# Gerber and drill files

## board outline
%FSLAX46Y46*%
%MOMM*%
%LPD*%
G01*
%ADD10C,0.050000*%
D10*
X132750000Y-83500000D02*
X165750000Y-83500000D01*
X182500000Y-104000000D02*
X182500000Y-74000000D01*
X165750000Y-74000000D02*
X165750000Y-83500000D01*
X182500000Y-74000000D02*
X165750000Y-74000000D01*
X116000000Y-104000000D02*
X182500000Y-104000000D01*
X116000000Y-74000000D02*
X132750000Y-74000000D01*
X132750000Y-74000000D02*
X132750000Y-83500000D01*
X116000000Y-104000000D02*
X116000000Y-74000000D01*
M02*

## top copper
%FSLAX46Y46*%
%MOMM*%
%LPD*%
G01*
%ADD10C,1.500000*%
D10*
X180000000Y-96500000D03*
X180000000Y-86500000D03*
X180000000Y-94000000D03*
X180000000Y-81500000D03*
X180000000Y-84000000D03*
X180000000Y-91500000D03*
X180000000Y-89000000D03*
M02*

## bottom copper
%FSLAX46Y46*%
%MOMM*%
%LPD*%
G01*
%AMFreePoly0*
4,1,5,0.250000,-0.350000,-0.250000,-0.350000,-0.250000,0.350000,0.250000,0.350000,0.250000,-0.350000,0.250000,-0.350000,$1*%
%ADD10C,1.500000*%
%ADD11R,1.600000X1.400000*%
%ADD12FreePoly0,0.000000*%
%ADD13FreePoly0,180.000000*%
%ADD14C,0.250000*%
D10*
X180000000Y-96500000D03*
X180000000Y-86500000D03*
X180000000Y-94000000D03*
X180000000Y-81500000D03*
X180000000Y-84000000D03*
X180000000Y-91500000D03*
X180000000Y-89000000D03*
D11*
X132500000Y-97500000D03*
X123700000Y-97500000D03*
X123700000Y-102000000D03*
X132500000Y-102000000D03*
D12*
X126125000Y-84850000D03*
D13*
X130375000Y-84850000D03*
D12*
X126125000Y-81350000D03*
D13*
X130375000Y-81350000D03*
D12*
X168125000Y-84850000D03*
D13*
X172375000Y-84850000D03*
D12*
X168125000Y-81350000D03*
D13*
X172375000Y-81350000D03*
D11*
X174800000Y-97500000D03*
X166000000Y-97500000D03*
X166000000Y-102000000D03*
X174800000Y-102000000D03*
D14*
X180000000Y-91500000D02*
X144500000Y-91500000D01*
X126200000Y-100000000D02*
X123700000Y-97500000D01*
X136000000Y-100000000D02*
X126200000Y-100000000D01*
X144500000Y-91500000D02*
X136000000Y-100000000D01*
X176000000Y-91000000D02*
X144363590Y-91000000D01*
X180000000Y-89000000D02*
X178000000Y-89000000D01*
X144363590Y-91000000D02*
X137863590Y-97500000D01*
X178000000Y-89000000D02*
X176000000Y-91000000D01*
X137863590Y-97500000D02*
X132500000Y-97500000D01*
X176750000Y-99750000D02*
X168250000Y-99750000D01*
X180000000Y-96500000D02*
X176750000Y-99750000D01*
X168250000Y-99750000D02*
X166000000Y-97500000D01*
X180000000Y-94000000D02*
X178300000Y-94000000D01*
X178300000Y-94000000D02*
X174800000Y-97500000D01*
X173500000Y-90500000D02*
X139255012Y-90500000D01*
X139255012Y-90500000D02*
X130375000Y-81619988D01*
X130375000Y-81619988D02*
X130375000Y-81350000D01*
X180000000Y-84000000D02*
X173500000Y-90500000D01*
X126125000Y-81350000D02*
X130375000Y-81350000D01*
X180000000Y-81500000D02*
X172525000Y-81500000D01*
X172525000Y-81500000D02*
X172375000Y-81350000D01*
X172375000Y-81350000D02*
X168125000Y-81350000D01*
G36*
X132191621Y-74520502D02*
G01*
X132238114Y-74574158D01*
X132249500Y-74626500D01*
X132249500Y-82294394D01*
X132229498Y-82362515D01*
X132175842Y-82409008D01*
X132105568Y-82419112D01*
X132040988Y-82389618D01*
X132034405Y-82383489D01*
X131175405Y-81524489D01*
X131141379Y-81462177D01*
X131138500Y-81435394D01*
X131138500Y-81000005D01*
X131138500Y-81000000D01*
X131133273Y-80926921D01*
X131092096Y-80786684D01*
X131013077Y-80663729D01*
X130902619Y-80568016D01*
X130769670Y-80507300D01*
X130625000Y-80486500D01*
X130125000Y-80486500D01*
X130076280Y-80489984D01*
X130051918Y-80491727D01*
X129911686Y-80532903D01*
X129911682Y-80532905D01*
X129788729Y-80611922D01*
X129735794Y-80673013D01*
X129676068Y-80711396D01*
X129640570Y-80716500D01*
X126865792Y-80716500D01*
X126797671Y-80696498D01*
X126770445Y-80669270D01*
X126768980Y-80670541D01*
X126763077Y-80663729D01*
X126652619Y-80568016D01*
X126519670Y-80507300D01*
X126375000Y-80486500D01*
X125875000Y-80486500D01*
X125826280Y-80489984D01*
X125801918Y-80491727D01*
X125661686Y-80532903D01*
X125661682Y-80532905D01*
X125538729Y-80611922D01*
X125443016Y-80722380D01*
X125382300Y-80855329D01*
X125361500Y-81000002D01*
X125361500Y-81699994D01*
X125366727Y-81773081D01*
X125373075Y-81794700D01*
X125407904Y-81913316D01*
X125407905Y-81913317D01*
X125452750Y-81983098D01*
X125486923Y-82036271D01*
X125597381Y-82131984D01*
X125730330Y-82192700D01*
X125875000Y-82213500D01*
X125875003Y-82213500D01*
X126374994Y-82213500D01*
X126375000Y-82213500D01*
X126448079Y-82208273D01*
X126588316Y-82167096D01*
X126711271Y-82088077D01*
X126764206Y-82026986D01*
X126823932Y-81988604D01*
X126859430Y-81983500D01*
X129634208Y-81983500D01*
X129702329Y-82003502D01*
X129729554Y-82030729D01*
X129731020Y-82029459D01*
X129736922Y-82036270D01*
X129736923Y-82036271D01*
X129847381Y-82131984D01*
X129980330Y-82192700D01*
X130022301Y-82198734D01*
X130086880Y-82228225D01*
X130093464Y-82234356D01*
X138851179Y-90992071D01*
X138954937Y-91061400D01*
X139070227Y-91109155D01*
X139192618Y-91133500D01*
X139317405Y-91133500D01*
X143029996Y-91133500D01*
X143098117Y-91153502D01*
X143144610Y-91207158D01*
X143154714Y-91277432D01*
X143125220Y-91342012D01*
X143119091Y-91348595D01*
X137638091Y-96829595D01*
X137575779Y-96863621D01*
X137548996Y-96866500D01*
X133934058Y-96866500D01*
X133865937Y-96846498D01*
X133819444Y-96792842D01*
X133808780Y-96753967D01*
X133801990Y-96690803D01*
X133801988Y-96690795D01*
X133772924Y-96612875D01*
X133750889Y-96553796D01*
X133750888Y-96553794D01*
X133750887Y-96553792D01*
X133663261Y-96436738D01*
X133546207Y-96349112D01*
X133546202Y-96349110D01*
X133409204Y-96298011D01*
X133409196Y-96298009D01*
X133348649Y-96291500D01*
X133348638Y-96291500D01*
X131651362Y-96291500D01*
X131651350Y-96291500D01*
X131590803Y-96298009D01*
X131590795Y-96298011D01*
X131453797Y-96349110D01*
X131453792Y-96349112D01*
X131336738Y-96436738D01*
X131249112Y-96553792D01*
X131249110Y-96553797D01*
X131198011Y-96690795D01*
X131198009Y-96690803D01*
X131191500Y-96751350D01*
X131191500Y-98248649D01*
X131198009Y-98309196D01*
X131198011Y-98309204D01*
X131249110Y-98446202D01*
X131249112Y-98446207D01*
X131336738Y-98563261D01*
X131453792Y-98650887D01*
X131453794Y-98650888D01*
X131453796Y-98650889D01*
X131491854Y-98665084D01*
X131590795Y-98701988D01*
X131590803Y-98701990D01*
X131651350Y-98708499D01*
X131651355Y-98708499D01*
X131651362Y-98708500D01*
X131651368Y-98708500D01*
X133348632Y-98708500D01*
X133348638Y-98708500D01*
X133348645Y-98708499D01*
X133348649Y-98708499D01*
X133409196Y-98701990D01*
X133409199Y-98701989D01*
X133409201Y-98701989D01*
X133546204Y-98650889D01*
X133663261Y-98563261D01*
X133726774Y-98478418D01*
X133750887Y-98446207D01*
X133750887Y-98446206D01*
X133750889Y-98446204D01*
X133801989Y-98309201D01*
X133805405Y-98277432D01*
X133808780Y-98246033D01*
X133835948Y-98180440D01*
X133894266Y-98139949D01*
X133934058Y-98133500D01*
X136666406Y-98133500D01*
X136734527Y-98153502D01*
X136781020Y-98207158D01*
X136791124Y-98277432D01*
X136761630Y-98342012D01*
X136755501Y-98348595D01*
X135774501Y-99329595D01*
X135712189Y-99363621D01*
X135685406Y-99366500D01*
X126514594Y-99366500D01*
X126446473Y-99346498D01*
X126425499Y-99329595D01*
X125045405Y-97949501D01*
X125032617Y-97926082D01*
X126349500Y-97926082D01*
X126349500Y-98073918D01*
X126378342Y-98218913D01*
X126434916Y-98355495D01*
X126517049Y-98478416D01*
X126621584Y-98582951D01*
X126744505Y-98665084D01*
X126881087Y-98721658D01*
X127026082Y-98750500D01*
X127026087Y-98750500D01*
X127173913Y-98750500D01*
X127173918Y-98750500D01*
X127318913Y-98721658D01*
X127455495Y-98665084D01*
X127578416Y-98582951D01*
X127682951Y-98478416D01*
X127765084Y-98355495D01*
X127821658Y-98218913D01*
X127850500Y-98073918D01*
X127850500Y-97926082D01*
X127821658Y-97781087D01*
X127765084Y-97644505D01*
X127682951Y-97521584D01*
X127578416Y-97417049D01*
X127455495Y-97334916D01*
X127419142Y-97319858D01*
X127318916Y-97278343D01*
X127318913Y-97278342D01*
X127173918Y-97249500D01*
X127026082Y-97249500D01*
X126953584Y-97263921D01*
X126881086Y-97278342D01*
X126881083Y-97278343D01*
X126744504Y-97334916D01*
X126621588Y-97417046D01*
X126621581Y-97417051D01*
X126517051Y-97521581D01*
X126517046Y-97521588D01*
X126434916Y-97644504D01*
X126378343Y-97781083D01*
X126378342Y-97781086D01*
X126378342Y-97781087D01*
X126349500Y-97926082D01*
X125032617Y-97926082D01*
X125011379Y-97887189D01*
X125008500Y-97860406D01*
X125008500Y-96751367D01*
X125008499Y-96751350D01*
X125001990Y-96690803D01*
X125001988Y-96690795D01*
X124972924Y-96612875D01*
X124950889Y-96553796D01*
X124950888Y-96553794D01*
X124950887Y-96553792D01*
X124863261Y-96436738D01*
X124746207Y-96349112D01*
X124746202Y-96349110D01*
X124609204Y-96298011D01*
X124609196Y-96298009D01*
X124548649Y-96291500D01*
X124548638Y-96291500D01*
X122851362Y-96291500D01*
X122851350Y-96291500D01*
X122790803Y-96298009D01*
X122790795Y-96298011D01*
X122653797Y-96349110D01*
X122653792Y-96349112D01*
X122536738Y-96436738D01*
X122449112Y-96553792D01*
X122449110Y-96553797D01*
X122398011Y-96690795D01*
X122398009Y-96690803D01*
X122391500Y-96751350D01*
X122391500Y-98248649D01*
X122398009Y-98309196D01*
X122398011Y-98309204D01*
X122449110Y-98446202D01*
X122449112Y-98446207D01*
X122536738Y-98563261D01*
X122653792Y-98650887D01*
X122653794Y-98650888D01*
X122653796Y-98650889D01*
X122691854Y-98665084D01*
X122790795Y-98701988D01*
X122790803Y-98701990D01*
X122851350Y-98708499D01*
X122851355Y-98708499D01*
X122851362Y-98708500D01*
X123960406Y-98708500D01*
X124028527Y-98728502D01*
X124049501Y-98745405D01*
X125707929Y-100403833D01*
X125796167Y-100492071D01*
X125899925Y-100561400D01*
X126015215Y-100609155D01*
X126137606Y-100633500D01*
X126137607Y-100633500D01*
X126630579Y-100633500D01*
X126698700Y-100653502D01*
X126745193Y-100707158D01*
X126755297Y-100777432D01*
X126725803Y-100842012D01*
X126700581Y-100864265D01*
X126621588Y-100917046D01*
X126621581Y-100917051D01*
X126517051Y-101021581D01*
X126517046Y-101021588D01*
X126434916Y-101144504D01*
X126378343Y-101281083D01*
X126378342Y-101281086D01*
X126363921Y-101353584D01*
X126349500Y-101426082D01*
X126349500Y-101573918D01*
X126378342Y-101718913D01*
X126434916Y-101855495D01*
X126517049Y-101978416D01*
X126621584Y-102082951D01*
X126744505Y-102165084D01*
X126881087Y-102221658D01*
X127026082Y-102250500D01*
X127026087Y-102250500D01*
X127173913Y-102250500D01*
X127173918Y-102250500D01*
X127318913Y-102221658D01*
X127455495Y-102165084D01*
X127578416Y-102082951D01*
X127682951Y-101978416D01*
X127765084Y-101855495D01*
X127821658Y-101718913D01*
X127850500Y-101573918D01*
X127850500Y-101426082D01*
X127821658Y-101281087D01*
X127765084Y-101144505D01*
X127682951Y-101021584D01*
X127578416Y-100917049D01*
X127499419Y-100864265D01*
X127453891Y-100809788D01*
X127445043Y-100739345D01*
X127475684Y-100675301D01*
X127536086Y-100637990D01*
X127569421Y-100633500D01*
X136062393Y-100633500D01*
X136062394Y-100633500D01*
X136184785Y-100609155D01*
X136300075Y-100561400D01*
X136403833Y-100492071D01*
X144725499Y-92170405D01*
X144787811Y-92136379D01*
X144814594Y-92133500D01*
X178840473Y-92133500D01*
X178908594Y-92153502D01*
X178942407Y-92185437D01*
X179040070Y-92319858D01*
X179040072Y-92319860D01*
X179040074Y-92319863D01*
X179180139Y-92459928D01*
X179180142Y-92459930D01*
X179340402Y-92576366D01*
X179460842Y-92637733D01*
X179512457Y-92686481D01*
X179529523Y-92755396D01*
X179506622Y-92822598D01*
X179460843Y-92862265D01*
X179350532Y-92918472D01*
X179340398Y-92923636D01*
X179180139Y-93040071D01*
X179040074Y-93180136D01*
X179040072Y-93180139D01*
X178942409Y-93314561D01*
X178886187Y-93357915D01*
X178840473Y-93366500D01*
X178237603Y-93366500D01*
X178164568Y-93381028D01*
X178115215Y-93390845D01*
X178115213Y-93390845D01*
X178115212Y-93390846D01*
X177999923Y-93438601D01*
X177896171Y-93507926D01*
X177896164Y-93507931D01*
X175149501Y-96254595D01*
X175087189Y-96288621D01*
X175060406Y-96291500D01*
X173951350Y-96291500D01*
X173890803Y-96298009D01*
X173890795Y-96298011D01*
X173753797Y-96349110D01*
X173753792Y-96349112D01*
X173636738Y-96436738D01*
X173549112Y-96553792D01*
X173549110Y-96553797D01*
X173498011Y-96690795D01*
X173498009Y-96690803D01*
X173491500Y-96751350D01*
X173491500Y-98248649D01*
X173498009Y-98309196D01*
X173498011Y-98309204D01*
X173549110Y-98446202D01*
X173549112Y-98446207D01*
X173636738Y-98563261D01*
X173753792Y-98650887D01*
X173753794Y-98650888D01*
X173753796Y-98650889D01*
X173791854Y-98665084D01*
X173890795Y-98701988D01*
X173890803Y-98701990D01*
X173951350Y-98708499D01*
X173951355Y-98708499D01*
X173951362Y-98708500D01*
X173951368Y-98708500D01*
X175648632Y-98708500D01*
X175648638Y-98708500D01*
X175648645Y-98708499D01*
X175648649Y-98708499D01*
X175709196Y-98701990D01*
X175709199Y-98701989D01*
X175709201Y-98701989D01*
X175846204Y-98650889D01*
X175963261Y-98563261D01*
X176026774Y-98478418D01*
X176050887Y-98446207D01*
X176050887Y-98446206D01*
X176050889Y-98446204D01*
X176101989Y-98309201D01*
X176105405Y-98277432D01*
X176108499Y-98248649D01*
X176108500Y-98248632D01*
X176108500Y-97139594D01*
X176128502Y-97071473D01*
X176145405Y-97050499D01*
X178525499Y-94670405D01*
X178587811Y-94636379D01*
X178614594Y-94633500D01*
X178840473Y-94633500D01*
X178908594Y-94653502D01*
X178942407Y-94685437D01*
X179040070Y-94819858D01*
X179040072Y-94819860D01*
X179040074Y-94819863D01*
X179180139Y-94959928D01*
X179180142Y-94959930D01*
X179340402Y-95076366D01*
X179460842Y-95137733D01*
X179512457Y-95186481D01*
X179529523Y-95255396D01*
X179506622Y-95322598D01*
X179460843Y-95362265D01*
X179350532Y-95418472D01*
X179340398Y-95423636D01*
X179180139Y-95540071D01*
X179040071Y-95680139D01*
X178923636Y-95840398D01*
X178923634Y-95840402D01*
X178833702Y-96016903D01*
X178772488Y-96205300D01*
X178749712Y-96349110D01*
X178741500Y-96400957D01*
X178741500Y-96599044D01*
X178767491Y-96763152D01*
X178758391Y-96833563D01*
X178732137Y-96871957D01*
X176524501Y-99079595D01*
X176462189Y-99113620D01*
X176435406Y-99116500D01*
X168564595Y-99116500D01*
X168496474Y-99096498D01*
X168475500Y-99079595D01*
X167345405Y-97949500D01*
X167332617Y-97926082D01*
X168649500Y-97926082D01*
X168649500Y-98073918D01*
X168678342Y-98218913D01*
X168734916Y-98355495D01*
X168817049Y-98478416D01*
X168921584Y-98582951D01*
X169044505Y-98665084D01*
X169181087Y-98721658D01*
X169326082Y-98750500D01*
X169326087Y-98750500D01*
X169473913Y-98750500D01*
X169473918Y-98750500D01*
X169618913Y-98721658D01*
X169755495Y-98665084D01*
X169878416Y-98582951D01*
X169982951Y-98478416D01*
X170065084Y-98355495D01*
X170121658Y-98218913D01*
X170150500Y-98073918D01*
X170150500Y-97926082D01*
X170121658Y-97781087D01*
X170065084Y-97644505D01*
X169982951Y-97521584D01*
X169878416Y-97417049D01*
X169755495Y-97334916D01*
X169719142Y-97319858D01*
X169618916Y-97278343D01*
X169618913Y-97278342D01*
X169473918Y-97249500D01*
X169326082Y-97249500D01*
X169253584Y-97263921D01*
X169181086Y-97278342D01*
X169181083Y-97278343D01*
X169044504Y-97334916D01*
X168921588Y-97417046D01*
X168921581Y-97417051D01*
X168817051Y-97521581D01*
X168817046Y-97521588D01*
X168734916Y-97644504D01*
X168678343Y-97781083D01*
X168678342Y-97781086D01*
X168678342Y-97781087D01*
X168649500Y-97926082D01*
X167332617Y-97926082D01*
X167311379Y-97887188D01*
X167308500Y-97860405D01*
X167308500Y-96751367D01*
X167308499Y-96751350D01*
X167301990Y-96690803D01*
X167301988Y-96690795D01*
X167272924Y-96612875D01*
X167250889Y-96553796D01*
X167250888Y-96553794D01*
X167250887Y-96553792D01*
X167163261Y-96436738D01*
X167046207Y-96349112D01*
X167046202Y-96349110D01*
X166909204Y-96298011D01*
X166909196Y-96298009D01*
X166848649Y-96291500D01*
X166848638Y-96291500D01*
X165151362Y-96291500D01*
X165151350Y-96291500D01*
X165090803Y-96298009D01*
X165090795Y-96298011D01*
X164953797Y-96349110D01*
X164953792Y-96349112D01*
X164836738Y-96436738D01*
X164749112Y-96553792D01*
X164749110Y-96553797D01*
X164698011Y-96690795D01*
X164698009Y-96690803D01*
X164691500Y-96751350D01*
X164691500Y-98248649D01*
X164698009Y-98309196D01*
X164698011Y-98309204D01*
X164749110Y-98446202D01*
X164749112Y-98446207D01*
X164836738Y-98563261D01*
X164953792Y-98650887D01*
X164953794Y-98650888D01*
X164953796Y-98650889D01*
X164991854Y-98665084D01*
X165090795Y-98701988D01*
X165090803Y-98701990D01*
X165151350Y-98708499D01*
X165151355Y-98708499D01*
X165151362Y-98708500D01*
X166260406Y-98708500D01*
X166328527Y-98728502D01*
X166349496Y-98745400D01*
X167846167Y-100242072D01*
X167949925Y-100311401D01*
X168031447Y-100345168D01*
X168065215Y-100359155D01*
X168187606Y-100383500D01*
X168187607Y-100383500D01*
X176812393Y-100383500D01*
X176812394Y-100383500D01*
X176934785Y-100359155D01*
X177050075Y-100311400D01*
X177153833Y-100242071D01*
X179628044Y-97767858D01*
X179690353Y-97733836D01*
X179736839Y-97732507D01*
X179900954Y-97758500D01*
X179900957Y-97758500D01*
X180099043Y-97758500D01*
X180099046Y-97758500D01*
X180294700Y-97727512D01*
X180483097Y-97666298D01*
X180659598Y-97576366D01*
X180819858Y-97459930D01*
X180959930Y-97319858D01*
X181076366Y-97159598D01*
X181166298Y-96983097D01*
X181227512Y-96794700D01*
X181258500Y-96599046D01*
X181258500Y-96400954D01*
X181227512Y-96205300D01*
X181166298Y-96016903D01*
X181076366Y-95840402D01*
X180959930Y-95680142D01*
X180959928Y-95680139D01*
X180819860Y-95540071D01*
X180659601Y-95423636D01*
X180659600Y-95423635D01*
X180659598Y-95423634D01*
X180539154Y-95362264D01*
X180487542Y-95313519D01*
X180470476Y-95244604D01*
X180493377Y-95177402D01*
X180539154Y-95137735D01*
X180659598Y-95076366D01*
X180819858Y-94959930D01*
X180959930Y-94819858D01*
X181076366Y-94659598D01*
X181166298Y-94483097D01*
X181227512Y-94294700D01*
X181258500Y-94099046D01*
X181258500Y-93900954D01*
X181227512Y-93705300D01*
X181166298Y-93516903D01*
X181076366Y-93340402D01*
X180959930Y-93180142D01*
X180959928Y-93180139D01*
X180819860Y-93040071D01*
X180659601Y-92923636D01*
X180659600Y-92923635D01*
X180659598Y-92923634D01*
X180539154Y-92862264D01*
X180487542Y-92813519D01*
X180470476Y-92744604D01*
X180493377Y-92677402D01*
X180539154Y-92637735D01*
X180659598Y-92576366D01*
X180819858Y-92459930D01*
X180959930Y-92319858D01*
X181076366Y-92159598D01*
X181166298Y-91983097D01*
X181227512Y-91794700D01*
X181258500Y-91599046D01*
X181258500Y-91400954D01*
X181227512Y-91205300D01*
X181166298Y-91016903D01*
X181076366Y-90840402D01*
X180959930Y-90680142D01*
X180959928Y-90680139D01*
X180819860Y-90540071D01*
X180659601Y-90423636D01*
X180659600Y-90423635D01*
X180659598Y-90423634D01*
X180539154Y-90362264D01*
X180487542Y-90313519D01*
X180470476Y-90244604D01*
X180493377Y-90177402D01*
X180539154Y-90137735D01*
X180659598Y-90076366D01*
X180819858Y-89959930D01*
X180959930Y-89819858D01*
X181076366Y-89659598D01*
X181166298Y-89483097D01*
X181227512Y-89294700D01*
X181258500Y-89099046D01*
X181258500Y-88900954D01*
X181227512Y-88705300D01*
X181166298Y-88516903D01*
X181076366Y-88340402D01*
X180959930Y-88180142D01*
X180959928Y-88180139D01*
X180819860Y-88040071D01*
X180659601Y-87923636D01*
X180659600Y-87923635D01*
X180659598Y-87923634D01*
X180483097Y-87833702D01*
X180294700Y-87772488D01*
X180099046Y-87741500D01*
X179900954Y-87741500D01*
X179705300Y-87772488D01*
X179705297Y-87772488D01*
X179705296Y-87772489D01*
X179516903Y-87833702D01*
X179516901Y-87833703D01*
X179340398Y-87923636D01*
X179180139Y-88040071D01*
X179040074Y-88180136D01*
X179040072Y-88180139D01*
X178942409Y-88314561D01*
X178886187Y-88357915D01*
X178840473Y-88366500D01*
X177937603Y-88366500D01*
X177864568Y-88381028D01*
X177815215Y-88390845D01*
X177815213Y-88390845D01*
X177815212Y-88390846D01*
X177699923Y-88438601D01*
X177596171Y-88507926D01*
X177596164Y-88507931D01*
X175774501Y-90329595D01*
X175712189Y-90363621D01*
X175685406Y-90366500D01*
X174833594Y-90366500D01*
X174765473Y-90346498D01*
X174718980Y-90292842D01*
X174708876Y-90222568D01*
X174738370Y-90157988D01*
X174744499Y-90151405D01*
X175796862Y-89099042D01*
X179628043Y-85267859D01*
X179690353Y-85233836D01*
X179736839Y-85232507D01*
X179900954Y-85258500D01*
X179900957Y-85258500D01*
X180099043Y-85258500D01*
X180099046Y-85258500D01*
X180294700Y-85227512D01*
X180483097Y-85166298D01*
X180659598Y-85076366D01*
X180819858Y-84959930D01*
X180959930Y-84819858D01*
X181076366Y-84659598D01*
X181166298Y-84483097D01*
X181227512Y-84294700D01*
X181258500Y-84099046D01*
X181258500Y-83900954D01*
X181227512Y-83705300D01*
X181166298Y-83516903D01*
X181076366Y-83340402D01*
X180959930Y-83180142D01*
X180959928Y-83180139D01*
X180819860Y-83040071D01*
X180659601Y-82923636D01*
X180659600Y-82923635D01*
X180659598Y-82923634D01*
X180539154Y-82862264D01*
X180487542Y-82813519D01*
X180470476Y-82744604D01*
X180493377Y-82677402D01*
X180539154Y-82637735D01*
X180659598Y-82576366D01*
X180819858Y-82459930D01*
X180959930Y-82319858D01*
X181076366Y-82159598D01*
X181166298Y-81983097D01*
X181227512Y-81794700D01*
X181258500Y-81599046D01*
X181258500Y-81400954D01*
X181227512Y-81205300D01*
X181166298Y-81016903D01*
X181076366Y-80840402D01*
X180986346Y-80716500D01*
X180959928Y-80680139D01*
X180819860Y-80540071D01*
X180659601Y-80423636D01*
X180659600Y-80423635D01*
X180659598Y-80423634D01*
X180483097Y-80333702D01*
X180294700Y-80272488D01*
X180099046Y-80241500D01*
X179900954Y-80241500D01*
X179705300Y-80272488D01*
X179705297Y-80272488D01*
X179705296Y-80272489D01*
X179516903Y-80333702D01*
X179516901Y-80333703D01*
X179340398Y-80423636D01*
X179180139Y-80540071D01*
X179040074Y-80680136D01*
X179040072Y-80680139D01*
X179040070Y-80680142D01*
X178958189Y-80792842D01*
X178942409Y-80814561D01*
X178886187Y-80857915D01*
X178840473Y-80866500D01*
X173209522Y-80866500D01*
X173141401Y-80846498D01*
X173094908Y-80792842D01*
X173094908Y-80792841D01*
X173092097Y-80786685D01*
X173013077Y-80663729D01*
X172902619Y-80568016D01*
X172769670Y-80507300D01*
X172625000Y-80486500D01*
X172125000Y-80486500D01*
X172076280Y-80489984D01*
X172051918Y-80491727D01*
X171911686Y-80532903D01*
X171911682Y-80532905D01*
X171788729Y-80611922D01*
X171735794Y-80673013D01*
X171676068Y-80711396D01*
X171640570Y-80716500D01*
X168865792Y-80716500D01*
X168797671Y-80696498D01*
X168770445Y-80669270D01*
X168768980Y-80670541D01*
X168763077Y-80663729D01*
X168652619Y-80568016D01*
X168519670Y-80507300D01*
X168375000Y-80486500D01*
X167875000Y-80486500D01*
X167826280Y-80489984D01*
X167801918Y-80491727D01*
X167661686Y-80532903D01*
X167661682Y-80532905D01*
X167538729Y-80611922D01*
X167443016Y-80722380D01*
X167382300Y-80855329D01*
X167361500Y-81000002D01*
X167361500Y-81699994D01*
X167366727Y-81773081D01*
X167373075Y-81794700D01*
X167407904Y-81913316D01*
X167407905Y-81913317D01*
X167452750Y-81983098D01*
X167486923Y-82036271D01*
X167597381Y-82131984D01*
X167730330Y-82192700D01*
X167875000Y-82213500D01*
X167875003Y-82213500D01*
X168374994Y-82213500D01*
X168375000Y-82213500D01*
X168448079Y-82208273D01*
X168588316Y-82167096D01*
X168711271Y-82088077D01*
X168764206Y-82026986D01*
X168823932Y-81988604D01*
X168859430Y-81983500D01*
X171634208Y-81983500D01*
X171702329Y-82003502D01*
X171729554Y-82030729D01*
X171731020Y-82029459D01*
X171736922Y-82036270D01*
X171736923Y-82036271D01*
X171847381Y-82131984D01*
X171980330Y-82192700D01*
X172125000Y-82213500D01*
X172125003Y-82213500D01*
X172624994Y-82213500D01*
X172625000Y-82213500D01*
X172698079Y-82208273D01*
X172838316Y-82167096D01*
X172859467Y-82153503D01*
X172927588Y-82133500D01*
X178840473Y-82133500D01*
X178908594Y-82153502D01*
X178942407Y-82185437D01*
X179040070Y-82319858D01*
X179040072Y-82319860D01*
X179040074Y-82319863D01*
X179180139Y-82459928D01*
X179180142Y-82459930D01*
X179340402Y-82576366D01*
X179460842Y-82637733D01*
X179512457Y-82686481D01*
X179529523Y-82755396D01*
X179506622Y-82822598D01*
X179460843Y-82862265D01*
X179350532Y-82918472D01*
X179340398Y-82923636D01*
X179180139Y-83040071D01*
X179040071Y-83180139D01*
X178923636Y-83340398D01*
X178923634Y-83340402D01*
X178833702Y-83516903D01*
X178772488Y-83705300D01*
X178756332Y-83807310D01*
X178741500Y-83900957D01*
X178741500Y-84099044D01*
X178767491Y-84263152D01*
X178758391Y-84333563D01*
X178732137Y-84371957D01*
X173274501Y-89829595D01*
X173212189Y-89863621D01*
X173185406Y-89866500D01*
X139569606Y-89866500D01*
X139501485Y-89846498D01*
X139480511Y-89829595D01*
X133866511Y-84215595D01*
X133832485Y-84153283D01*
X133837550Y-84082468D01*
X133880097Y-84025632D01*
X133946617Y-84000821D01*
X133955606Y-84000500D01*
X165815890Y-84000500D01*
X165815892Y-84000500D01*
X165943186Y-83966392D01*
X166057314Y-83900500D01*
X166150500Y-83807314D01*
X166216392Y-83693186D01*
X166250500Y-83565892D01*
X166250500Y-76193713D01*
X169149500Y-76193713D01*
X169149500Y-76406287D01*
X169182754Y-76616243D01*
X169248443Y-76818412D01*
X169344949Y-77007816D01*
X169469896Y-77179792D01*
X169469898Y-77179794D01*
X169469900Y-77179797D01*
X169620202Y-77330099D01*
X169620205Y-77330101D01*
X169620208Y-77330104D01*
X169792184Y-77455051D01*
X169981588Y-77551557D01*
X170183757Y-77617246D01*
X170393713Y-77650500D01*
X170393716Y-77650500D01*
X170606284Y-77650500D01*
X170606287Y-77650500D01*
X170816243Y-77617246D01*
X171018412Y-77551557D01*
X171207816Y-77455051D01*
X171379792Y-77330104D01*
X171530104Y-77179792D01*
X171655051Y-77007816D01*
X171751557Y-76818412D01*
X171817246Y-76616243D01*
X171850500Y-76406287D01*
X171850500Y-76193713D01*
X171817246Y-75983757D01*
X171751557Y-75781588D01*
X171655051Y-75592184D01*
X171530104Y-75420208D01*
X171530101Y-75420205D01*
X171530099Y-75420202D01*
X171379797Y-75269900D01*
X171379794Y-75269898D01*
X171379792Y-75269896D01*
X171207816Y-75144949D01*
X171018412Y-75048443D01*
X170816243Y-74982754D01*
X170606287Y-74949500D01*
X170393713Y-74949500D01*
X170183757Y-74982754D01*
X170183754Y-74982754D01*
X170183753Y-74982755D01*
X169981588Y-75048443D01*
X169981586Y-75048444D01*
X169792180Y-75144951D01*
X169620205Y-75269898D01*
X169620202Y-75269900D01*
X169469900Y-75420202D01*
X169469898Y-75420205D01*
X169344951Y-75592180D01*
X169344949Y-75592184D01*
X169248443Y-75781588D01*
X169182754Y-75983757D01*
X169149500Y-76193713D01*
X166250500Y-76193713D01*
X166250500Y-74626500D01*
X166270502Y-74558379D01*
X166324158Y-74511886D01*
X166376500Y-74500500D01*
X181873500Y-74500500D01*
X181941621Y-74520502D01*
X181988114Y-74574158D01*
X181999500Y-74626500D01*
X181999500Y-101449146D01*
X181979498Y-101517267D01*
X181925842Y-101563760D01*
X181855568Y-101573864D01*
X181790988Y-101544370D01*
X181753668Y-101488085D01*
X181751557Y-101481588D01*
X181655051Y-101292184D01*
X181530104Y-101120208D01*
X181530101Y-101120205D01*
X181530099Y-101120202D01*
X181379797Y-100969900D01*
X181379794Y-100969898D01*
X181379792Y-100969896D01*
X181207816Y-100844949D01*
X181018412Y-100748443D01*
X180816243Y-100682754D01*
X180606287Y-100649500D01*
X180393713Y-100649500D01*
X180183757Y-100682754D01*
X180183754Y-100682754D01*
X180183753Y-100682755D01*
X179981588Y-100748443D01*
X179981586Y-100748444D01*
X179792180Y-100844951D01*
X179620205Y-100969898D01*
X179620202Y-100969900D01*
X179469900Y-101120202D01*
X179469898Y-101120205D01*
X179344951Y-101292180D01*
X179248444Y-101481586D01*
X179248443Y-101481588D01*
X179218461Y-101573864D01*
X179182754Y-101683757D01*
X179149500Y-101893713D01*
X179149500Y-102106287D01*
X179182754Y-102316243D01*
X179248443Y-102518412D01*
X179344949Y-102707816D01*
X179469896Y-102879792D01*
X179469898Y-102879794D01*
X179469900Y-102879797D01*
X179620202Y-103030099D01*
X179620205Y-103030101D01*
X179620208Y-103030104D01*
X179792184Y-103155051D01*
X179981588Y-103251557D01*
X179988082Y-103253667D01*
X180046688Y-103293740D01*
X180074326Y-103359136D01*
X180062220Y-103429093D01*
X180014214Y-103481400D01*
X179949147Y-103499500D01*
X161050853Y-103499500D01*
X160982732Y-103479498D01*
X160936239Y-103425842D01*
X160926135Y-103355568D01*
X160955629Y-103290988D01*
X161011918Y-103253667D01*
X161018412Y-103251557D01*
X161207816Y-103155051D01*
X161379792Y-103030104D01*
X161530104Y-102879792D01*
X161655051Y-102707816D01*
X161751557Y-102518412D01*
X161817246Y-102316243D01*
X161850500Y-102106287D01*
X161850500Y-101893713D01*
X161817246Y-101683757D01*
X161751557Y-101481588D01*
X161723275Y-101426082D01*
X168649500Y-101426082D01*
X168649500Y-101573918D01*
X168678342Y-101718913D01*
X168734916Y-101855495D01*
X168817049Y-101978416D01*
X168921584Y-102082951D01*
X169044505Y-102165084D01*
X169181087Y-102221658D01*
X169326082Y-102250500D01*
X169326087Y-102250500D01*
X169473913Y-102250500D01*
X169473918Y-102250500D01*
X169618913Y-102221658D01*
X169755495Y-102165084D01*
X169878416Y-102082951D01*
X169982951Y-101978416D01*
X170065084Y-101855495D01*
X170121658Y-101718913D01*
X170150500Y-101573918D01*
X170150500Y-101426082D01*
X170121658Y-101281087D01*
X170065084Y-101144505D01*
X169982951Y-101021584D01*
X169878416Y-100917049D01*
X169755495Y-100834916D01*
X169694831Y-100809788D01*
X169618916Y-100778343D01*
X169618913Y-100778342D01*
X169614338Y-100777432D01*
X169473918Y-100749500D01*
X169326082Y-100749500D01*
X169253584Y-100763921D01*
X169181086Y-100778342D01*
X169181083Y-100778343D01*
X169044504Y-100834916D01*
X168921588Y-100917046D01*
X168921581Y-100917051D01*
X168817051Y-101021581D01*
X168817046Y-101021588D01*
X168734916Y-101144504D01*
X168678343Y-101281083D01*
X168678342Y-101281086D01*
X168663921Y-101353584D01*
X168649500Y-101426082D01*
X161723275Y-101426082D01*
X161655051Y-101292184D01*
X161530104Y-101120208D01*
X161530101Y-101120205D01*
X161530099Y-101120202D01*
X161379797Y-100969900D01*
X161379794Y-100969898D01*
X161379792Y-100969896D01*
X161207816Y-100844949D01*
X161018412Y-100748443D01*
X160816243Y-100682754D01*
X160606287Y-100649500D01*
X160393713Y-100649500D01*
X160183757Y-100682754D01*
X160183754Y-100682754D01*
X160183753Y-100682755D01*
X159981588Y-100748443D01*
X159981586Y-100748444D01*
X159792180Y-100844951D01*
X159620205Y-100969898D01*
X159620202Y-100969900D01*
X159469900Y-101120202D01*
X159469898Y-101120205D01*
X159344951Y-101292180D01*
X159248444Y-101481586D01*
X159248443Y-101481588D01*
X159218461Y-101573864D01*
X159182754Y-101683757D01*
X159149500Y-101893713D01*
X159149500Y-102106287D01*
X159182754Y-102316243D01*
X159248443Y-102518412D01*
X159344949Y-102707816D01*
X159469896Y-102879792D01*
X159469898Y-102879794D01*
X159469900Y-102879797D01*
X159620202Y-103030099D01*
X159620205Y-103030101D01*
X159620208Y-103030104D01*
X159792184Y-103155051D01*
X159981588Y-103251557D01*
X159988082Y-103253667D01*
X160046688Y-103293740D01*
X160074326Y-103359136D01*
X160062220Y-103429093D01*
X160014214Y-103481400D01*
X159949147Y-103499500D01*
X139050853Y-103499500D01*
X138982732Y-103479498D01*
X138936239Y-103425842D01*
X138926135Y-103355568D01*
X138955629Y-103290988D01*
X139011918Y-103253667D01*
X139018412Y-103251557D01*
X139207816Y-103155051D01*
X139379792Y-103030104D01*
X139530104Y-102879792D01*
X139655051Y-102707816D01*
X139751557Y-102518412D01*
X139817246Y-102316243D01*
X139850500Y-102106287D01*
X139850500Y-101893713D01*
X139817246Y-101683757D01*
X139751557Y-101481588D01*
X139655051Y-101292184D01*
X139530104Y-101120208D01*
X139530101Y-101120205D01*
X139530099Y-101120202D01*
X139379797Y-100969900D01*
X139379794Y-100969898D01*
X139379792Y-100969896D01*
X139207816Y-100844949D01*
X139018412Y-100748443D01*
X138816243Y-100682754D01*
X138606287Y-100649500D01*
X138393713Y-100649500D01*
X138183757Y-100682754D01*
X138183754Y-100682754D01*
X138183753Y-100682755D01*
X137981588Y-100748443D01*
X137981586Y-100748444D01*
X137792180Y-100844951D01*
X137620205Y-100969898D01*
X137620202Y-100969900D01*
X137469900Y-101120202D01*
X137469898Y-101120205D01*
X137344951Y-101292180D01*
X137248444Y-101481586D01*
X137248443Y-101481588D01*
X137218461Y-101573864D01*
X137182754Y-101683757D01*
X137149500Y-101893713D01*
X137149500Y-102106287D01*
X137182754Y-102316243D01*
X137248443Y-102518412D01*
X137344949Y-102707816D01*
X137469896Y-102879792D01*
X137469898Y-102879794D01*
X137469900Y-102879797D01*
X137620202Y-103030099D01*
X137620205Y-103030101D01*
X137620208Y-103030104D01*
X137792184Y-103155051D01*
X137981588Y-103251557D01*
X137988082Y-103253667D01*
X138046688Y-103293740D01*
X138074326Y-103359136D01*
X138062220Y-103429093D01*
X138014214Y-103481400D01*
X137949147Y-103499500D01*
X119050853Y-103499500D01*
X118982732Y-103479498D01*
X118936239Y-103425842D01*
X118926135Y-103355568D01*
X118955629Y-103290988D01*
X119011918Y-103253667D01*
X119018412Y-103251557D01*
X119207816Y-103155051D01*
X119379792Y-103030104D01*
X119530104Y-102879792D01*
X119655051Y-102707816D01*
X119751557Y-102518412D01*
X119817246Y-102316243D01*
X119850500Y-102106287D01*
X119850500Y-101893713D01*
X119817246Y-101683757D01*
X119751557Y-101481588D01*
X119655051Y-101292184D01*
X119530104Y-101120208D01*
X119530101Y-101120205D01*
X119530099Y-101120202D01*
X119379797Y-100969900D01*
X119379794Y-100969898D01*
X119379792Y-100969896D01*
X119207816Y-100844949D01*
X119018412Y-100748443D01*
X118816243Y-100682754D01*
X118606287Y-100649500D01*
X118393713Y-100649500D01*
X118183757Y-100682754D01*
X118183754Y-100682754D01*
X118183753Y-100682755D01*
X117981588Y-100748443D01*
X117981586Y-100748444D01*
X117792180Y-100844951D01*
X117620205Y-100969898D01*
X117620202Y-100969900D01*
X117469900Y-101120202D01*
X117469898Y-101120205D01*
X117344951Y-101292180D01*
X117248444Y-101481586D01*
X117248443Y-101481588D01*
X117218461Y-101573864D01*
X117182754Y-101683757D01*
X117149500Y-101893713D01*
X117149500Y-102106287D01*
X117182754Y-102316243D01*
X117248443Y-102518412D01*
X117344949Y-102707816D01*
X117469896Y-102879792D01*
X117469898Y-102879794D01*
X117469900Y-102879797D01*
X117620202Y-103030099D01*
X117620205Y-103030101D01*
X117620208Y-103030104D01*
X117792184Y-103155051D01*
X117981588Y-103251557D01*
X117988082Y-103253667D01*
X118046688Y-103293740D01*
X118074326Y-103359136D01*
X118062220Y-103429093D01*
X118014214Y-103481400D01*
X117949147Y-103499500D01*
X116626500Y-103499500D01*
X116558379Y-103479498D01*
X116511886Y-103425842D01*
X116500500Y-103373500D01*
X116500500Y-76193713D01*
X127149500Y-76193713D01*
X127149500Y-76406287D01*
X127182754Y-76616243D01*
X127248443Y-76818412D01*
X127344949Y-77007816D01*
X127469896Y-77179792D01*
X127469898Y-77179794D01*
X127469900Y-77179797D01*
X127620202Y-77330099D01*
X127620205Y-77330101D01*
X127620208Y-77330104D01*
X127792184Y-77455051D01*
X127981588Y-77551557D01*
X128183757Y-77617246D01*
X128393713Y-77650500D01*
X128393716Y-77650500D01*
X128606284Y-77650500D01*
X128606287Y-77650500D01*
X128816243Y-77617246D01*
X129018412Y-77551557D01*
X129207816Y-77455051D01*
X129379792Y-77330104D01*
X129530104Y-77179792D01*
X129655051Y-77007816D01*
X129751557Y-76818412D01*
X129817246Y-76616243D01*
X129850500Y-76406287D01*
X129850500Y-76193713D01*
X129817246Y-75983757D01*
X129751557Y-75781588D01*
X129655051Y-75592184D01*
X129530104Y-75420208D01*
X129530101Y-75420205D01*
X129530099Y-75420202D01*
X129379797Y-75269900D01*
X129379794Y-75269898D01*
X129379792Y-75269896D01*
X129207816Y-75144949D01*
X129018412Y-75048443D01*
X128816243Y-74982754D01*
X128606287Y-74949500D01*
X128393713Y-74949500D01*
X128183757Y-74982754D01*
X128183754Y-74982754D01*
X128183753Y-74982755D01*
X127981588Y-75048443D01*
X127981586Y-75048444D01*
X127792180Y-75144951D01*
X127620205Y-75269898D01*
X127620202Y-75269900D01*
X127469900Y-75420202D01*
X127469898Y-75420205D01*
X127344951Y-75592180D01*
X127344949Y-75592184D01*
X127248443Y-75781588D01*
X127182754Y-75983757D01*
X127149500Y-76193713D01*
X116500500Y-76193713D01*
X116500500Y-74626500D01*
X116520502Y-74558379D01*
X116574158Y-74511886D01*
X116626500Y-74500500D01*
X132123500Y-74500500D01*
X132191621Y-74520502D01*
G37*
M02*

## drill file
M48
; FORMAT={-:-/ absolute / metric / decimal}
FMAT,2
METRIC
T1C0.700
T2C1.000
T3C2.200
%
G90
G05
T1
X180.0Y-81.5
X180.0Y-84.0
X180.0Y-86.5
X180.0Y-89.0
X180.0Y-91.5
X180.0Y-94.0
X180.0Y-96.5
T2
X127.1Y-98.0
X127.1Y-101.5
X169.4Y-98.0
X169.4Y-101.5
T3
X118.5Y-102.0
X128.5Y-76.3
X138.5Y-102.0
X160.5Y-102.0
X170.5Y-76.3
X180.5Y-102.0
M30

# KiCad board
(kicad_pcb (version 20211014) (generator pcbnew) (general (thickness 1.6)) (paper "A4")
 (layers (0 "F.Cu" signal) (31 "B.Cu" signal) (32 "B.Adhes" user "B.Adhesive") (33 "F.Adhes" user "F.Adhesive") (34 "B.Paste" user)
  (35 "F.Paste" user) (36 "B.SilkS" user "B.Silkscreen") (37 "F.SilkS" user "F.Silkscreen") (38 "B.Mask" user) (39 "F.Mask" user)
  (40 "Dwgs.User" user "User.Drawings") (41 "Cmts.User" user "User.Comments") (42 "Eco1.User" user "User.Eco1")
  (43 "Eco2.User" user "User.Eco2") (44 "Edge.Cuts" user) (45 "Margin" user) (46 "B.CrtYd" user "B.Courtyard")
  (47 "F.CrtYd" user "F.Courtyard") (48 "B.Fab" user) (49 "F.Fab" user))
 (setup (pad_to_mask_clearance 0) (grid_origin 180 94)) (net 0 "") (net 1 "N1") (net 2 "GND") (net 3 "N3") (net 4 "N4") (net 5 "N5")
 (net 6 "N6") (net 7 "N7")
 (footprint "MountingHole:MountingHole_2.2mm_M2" (layer "F.Cu") (at 138.5 102)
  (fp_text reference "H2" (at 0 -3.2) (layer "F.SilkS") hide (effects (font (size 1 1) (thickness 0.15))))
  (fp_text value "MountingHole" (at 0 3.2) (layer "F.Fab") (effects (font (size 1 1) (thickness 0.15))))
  (pad "" np_thru_hole circle locked (at 0 0) (size 2.2 2.2) (drill 2.2) (layers *.Cu *.Mask)))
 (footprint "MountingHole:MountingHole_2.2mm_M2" (layer "F.Cu") (at 160.5 102)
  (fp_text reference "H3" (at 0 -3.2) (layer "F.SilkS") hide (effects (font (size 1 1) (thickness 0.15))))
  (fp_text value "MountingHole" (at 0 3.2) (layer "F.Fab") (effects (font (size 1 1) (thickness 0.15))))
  (pad "" np_thru_hole circle locked (at 0 0) (size 2.2 2.2) (drill 2.2) (layers *.Cu *.Mask)))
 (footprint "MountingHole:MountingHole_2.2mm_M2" (layer "F.Cu") (at 170.5 76.3)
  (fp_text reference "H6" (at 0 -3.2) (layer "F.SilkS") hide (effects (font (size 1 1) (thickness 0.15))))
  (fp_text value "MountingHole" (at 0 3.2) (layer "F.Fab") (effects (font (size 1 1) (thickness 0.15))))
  (pad "" np_thru_hole circle locked (at 0 0) (size 2.2 2.2) (drill 2.2) (layers *.Cu *.Mask)))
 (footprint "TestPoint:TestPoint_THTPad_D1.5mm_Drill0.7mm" (layer "F.Cu") (at 180 96.5)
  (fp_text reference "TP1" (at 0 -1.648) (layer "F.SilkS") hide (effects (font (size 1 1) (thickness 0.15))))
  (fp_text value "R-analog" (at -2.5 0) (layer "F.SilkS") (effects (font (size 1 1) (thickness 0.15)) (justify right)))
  (pad "1" thru_hole circle locked (at 0 0) (size 1.5 1.5) (drill 0.7) (layers *.Cu *.Mask) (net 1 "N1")))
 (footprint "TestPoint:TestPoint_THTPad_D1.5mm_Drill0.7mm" (layer "F.Cu") (at 180 86.5)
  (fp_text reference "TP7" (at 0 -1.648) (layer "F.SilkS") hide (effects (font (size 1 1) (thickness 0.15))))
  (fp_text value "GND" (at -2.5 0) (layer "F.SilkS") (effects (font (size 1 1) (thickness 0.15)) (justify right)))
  (pad "1" thru_hole circle locked (at 0 0) (size 1.5 1.5) (drill 0.7) (layers *.Cu *.Mask) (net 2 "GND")))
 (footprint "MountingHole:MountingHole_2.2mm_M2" (layer "F.Cu") (at 118.5 102)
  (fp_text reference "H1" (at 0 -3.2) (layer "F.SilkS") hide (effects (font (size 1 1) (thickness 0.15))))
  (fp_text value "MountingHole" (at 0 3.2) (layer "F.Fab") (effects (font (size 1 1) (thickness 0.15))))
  (pad "" np_thru_hole circle locked (at 0 0) (size 2.2 2.2) (drill 2.2) (layers *.Cu *.Mask)))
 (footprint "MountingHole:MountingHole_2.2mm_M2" (layer "F.Cu") (at 180.5 102)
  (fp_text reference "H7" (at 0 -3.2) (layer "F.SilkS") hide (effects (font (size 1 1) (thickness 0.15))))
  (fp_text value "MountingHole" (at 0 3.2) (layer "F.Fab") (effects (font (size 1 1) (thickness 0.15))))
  (pad "" np_thru_hole circle locked (at 0 0) (size 2.2 2.2) (drill 2.2) (layers *.Cu *.Mask)))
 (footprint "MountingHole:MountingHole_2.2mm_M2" (layer "F.Cu") (at 128.5 76.3)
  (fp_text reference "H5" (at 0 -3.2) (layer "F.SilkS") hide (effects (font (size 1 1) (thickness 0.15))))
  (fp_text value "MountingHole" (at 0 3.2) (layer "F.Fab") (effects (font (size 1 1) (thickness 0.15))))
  (pad "" np_thru_hole circle locked (at 0 0) (size 2.2 2.2) (drill 2.2) (layers *.Cu *.Mask)))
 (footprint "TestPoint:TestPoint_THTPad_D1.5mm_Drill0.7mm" (layer "F.Cu") (at 180 94)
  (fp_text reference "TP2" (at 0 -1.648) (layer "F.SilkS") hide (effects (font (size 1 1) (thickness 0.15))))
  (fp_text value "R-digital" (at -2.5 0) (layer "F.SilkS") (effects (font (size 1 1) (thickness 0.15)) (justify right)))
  (pad "1" thru_hole circle locked (at 0 0) (size 1.5 1.5) (drill 0.7) (layers *.Cu *.Mask) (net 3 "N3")))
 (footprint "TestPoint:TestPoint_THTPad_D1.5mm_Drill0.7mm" (layer "F.Cu") (at 180 81.5)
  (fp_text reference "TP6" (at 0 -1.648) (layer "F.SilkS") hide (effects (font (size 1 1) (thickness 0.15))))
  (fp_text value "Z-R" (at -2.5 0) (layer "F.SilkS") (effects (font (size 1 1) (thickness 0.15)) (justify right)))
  (pad "1" thru_hole circle locked (at 0 0) (size 1.5 1.5) (drill 0.7) (layers *.Cu *.Mask) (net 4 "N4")))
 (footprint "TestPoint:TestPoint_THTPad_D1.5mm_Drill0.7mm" (layer "F.Cu") (at 180 84)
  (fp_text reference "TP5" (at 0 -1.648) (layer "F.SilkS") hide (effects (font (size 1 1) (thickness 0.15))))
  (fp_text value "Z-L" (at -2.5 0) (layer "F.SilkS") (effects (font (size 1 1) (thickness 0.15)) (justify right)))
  (pad "1" thru_hole circle locked (at 0 0) (size 1.5 1.5) (drill 0.7) (layers *.Cu *.Mask) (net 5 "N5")))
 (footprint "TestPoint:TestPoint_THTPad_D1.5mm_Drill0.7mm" (layer "F.Cu") (at 180 91.5)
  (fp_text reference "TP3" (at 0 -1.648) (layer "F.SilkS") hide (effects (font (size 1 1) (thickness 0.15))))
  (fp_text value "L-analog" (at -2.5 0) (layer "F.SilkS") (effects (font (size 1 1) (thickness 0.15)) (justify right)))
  (pad "1" thru_hole circle locked (at 0 0) (size 1.5 1.5) (drill 0.7) (layers *.Cu *.Mask) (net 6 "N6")))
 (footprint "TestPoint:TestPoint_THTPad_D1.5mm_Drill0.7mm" (layer "F.Cu") (at 180 89)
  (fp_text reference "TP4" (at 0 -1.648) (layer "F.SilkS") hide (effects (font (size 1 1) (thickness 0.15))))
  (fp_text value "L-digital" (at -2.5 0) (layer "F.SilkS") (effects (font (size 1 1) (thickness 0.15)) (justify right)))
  (pad "1" thru_hole circle locked (at 0 0) (size 1.5 1.5) (drill 0.7) (layers *.Cu *.Mask) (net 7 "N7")))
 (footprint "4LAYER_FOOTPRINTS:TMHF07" (layer "B.Cu") (at 133.3 102.7 180)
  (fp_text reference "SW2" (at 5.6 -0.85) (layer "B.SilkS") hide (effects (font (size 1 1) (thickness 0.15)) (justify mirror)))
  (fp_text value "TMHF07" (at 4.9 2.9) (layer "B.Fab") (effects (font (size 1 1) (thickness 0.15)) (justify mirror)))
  (pad "" np_thru_hole circle locked (at 6.2 1.2 180) (size 1 1) (drill 1) (layers *.Cu *.Mask))
  (pad "" np_thru_hole circle locked (at 6.2 4.7 180) (size 1 1) (drill 1) (layers *.Cu *.Mask))
  (pad "1" smd rect locked (at 0.8 5.2 180) (size 1.6 1.4) (layers "B.Cu" "B.Paste" "B.Mask") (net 7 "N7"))
  (pad "2" smd rect locked (at 9.6 5.2 180) (size 1.6 1.4) (layers "B.Cu" "B.Paste" "B.Mask") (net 6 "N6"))
  (pad "C" smd rect locked (at 9.6 0.7 180) (size 1.6 1.4) (layers "B.Cu" "B.Paste" "B.Mask") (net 2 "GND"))
  (pad "D" smd rect locked (at 0.8 0.7 180) (size 1.6 1.4) (layers "B.Cu" "B.Paste" "B.Mask") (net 2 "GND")))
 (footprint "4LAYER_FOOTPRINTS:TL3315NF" (layer "B.Cu") (at 125.675 80.8)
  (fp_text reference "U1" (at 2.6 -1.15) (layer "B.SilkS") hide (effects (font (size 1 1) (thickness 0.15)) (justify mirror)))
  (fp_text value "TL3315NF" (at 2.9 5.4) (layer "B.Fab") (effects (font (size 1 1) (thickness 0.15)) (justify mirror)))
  (pad "1" smd custom locked (at 0.45 4.05) (size 0.5 0.7) (layers "B.Cu" "B.Paste" "B.Mask") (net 2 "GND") (zone_connect 2)
   (options (clearance outline) (anchor rect)) (primitives))
  (pad "2" smd custom locked (at 4.7 4.05 180) (size 0.5 0.7) (layers "B.Cu" "B.Paste" "B.Mask") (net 2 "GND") (zone_connect 2)
   (options (clearance outline) (anchor rect)) (primitives))
  (pad "3" smd custom locked (at 0.45 0.55) (size 0.5 0.7) (layers "B.Cu" "B.Paste" "B.Mask") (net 5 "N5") (zone_connect 2)
   (options (clearance outline) (anchor rect)) (primitives))
  (pad "4" smd custom locked (at 4.7 0.55 180) (size 0.5 0.7) (layers "B.Cu" "B.Paste" "B.Mask") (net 5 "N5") (zone_connect 2)
   (options (clearance outline) (anchor rect)) (primitives)))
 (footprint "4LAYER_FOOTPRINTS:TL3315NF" (layer "B.Cu") (at 167.675 80.8)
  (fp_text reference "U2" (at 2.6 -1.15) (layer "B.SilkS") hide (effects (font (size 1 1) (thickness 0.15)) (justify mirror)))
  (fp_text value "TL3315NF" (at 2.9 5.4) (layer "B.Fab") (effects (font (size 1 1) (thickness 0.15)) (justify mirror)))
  (pad "1" smd custom locked (at 0.45 4.05) (size 0.5 0.7) (layers "B.Cu" "B.Paste" "B.Mask") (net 2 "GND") (zone_connect 2)
   (options (clearance outline) (anchor rect)) (primitives))
  (pad "2" smd custom locked (at 4.7 4.05 180) (size 0.5 0.7) (layers "B.Cu" "B.Paste" "B.Mask") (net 2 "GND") (zone_connect 2)
   (options (clearance outline) (anchor rect)) (primitives))
  (pad "3" smd custom locked (at 0.45 0.55) (size 0.5 0.7) (layers "B.Cu" "B.Paste" "B.Mask") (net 4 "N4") (zone_connect 2)
   (options (clearance outline) (anchor rect)) (primitives))
  (pad "4" smd custom locked (at 4.7 0.55 180) (size 0.5 0.7) (layers "B.Cu" "B.Paste" "B.Mask") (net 4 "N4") (zone_connect 2)
   (options (clearance outline) (anchor rect)) (primitives)))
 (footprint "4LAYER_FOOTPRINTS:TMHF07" (layer "B.Cu") (at 175.6 102.7 180)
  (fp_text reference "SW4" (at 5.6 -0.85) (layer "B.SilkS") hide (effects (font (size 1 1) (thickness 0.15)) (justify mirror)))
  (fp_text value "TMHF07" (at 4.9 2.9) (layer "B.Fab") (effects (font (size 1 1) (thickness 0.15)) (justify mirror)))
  (pad "" np_thru_hole circle locked (at 6.2 4.7 180) (size 1 1) (drill 1) (layers *.Cu *.Mask))
  (pad "" np_thru_hole circle locked (at 6.2 1.2 180) (size 1 1) (drill 1) (layers *.Cu *.Mask))
  (pad "1" smd rect locked (at 0.8 5.2 180) (size 1.6 1.4) (layers "B.Cu" "B.Paste" "B.Mask") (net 3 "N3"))
  (pad "2" smd rect locked (at 9.6 5.2 180) (size 1.6 1.4) (layers "B.Cu" "B.Paste" "B.Mask") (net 1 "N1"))
  (pad "C" smd rect locked (at 9.6 0.7 180) (size 1.6 1.4) (layers "B.Cu" "B.Paste" "B.Mask") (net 2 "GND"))
  (pad "D" smd rect locked (at 0.8 0.7 180) (size 1.6 1.4) (layers "B.Cu" "B.Paste" "B.Mask") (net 2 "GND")))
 (gr_line (start 132.75 83.5) (end 165.75 83.5) (layer "Edge.Cuts") (width 0.05))
 (gr_line (start 182.5 104) (end 182.5 74) (layer "Edge.Cuts") (width 0.05))
 (gr_line (start 165.75 74) (end 165.75 83.5) (layer "Edge.Cuts") (width 0.05))
 (gr_line (start 182.5 74) (end 165.75 74) (layer "Edge.Cuts") (width 0.05))
 (gr_line (start 116 104) (end 182.5 104) (layer "Edge.Cuts") (width 0.05))
 (gr_line (start 116 74) (end 132.75 74) (layer "Edge.Cuts") (width 0.05))
 (gr_line (start 132.75 74) (end 132.75 83.5) (layer "Edge.Cuts") (width 0.05))
 (gr_line (start 116 104) (end 116 74) (layer "Edge.Cuts") (width 0.05))
 (segment (start 180 91.5) (end 144.5 91.5) (width 0.25) (layer "B.Cu") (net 6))
 (segment (start 126.2 100) (end 123.7 97.5) (width 0.25) (layer "B.Cu") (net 6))
 (segment (start 136 100) (end 126.2 100) (width 0.25) (layer "B.Cu") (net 6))
 (segment (start 144.5 91.5) (end 136 100) (width 0.25) (layer "B.Cu") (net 6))
 (segment (start 176 91) (end 144.36359 91) (width 0.25) (layer "B.Cu") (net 7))
 (segment (start 180 89) (end 178 89) (width 0.25) (layer "B.Cu") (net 7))
 (segment (start 144.36359 91) (end 137.86359 97.5) (width 0.25) (layer "B.Cu") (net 7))
 (segment (start 178 89) (end 176 91) (width 0.25) (layer "B.Cu") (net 7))
 (segment (start 137.86359 97.5) (end 132.5 97.5) (width 0.25) (layer "B.Cu") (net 7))
 (segment (start 176.75 99.75) (end 168.25 99.75) (width 0.25) (layer "B.Cu") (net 1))
 (segment (start 180 96.5) (end 176.75 99.75) (width 0.25) (layer "B.Cu") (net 1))
 (segment (start 168.25 99.75) (end 166 97.5) (width 0.25) (layer "B.Cu") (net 1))
 (segment (start 180 94) (end 178.3 94) (width 0.25) (layer "B.Cu") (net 3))
 (segment (start 178.3 94) (end 174.8 97.5) (width 0.25) (layer "B.Cu") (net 3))
 (segment (start 173.5 90.5) (end 139.255012 90.5) (width 0.25) (layer "B.Cu") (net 5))
 (segment (start 139.255012 90.5) (end 130.375 81.619988) (width 0.25) (layer "B.Cu") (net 5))
 (segment (start 130.375 81.619988) (end 130.375 81.35) (width 0.25) (layer "B.Cu") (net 5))
 (segment (start 180 84) (end 173.5 90.5) (width 0.25) (layer "B.Cu") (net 5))
 (segment (start 126.125 81.35) (end 130.375 81.35) (width 0.25) (layer "B.Cu") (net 5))
 (segment (start 180 81.5) (end 172.525 81.5) (width 0.25) (layer "B.Cu") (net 4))
 (segment (start 172.525 81.5) (end 172.375 81.35) (width 0.25) (layer "B.Cu") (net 4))
 (segment (start 172.375 81.35) (end 168.125 81.35) (width 0.25) (layer "B.Cu") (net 4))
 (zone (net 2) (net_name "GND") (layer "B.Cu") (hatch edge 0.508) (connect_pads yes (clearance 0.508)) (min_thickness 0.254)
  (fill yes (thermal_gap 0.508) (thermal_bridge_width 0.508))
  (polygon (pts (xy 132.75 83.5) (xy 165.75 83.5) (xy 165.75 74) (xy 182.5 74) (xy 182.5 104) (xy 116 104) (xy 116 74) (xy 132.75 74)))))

